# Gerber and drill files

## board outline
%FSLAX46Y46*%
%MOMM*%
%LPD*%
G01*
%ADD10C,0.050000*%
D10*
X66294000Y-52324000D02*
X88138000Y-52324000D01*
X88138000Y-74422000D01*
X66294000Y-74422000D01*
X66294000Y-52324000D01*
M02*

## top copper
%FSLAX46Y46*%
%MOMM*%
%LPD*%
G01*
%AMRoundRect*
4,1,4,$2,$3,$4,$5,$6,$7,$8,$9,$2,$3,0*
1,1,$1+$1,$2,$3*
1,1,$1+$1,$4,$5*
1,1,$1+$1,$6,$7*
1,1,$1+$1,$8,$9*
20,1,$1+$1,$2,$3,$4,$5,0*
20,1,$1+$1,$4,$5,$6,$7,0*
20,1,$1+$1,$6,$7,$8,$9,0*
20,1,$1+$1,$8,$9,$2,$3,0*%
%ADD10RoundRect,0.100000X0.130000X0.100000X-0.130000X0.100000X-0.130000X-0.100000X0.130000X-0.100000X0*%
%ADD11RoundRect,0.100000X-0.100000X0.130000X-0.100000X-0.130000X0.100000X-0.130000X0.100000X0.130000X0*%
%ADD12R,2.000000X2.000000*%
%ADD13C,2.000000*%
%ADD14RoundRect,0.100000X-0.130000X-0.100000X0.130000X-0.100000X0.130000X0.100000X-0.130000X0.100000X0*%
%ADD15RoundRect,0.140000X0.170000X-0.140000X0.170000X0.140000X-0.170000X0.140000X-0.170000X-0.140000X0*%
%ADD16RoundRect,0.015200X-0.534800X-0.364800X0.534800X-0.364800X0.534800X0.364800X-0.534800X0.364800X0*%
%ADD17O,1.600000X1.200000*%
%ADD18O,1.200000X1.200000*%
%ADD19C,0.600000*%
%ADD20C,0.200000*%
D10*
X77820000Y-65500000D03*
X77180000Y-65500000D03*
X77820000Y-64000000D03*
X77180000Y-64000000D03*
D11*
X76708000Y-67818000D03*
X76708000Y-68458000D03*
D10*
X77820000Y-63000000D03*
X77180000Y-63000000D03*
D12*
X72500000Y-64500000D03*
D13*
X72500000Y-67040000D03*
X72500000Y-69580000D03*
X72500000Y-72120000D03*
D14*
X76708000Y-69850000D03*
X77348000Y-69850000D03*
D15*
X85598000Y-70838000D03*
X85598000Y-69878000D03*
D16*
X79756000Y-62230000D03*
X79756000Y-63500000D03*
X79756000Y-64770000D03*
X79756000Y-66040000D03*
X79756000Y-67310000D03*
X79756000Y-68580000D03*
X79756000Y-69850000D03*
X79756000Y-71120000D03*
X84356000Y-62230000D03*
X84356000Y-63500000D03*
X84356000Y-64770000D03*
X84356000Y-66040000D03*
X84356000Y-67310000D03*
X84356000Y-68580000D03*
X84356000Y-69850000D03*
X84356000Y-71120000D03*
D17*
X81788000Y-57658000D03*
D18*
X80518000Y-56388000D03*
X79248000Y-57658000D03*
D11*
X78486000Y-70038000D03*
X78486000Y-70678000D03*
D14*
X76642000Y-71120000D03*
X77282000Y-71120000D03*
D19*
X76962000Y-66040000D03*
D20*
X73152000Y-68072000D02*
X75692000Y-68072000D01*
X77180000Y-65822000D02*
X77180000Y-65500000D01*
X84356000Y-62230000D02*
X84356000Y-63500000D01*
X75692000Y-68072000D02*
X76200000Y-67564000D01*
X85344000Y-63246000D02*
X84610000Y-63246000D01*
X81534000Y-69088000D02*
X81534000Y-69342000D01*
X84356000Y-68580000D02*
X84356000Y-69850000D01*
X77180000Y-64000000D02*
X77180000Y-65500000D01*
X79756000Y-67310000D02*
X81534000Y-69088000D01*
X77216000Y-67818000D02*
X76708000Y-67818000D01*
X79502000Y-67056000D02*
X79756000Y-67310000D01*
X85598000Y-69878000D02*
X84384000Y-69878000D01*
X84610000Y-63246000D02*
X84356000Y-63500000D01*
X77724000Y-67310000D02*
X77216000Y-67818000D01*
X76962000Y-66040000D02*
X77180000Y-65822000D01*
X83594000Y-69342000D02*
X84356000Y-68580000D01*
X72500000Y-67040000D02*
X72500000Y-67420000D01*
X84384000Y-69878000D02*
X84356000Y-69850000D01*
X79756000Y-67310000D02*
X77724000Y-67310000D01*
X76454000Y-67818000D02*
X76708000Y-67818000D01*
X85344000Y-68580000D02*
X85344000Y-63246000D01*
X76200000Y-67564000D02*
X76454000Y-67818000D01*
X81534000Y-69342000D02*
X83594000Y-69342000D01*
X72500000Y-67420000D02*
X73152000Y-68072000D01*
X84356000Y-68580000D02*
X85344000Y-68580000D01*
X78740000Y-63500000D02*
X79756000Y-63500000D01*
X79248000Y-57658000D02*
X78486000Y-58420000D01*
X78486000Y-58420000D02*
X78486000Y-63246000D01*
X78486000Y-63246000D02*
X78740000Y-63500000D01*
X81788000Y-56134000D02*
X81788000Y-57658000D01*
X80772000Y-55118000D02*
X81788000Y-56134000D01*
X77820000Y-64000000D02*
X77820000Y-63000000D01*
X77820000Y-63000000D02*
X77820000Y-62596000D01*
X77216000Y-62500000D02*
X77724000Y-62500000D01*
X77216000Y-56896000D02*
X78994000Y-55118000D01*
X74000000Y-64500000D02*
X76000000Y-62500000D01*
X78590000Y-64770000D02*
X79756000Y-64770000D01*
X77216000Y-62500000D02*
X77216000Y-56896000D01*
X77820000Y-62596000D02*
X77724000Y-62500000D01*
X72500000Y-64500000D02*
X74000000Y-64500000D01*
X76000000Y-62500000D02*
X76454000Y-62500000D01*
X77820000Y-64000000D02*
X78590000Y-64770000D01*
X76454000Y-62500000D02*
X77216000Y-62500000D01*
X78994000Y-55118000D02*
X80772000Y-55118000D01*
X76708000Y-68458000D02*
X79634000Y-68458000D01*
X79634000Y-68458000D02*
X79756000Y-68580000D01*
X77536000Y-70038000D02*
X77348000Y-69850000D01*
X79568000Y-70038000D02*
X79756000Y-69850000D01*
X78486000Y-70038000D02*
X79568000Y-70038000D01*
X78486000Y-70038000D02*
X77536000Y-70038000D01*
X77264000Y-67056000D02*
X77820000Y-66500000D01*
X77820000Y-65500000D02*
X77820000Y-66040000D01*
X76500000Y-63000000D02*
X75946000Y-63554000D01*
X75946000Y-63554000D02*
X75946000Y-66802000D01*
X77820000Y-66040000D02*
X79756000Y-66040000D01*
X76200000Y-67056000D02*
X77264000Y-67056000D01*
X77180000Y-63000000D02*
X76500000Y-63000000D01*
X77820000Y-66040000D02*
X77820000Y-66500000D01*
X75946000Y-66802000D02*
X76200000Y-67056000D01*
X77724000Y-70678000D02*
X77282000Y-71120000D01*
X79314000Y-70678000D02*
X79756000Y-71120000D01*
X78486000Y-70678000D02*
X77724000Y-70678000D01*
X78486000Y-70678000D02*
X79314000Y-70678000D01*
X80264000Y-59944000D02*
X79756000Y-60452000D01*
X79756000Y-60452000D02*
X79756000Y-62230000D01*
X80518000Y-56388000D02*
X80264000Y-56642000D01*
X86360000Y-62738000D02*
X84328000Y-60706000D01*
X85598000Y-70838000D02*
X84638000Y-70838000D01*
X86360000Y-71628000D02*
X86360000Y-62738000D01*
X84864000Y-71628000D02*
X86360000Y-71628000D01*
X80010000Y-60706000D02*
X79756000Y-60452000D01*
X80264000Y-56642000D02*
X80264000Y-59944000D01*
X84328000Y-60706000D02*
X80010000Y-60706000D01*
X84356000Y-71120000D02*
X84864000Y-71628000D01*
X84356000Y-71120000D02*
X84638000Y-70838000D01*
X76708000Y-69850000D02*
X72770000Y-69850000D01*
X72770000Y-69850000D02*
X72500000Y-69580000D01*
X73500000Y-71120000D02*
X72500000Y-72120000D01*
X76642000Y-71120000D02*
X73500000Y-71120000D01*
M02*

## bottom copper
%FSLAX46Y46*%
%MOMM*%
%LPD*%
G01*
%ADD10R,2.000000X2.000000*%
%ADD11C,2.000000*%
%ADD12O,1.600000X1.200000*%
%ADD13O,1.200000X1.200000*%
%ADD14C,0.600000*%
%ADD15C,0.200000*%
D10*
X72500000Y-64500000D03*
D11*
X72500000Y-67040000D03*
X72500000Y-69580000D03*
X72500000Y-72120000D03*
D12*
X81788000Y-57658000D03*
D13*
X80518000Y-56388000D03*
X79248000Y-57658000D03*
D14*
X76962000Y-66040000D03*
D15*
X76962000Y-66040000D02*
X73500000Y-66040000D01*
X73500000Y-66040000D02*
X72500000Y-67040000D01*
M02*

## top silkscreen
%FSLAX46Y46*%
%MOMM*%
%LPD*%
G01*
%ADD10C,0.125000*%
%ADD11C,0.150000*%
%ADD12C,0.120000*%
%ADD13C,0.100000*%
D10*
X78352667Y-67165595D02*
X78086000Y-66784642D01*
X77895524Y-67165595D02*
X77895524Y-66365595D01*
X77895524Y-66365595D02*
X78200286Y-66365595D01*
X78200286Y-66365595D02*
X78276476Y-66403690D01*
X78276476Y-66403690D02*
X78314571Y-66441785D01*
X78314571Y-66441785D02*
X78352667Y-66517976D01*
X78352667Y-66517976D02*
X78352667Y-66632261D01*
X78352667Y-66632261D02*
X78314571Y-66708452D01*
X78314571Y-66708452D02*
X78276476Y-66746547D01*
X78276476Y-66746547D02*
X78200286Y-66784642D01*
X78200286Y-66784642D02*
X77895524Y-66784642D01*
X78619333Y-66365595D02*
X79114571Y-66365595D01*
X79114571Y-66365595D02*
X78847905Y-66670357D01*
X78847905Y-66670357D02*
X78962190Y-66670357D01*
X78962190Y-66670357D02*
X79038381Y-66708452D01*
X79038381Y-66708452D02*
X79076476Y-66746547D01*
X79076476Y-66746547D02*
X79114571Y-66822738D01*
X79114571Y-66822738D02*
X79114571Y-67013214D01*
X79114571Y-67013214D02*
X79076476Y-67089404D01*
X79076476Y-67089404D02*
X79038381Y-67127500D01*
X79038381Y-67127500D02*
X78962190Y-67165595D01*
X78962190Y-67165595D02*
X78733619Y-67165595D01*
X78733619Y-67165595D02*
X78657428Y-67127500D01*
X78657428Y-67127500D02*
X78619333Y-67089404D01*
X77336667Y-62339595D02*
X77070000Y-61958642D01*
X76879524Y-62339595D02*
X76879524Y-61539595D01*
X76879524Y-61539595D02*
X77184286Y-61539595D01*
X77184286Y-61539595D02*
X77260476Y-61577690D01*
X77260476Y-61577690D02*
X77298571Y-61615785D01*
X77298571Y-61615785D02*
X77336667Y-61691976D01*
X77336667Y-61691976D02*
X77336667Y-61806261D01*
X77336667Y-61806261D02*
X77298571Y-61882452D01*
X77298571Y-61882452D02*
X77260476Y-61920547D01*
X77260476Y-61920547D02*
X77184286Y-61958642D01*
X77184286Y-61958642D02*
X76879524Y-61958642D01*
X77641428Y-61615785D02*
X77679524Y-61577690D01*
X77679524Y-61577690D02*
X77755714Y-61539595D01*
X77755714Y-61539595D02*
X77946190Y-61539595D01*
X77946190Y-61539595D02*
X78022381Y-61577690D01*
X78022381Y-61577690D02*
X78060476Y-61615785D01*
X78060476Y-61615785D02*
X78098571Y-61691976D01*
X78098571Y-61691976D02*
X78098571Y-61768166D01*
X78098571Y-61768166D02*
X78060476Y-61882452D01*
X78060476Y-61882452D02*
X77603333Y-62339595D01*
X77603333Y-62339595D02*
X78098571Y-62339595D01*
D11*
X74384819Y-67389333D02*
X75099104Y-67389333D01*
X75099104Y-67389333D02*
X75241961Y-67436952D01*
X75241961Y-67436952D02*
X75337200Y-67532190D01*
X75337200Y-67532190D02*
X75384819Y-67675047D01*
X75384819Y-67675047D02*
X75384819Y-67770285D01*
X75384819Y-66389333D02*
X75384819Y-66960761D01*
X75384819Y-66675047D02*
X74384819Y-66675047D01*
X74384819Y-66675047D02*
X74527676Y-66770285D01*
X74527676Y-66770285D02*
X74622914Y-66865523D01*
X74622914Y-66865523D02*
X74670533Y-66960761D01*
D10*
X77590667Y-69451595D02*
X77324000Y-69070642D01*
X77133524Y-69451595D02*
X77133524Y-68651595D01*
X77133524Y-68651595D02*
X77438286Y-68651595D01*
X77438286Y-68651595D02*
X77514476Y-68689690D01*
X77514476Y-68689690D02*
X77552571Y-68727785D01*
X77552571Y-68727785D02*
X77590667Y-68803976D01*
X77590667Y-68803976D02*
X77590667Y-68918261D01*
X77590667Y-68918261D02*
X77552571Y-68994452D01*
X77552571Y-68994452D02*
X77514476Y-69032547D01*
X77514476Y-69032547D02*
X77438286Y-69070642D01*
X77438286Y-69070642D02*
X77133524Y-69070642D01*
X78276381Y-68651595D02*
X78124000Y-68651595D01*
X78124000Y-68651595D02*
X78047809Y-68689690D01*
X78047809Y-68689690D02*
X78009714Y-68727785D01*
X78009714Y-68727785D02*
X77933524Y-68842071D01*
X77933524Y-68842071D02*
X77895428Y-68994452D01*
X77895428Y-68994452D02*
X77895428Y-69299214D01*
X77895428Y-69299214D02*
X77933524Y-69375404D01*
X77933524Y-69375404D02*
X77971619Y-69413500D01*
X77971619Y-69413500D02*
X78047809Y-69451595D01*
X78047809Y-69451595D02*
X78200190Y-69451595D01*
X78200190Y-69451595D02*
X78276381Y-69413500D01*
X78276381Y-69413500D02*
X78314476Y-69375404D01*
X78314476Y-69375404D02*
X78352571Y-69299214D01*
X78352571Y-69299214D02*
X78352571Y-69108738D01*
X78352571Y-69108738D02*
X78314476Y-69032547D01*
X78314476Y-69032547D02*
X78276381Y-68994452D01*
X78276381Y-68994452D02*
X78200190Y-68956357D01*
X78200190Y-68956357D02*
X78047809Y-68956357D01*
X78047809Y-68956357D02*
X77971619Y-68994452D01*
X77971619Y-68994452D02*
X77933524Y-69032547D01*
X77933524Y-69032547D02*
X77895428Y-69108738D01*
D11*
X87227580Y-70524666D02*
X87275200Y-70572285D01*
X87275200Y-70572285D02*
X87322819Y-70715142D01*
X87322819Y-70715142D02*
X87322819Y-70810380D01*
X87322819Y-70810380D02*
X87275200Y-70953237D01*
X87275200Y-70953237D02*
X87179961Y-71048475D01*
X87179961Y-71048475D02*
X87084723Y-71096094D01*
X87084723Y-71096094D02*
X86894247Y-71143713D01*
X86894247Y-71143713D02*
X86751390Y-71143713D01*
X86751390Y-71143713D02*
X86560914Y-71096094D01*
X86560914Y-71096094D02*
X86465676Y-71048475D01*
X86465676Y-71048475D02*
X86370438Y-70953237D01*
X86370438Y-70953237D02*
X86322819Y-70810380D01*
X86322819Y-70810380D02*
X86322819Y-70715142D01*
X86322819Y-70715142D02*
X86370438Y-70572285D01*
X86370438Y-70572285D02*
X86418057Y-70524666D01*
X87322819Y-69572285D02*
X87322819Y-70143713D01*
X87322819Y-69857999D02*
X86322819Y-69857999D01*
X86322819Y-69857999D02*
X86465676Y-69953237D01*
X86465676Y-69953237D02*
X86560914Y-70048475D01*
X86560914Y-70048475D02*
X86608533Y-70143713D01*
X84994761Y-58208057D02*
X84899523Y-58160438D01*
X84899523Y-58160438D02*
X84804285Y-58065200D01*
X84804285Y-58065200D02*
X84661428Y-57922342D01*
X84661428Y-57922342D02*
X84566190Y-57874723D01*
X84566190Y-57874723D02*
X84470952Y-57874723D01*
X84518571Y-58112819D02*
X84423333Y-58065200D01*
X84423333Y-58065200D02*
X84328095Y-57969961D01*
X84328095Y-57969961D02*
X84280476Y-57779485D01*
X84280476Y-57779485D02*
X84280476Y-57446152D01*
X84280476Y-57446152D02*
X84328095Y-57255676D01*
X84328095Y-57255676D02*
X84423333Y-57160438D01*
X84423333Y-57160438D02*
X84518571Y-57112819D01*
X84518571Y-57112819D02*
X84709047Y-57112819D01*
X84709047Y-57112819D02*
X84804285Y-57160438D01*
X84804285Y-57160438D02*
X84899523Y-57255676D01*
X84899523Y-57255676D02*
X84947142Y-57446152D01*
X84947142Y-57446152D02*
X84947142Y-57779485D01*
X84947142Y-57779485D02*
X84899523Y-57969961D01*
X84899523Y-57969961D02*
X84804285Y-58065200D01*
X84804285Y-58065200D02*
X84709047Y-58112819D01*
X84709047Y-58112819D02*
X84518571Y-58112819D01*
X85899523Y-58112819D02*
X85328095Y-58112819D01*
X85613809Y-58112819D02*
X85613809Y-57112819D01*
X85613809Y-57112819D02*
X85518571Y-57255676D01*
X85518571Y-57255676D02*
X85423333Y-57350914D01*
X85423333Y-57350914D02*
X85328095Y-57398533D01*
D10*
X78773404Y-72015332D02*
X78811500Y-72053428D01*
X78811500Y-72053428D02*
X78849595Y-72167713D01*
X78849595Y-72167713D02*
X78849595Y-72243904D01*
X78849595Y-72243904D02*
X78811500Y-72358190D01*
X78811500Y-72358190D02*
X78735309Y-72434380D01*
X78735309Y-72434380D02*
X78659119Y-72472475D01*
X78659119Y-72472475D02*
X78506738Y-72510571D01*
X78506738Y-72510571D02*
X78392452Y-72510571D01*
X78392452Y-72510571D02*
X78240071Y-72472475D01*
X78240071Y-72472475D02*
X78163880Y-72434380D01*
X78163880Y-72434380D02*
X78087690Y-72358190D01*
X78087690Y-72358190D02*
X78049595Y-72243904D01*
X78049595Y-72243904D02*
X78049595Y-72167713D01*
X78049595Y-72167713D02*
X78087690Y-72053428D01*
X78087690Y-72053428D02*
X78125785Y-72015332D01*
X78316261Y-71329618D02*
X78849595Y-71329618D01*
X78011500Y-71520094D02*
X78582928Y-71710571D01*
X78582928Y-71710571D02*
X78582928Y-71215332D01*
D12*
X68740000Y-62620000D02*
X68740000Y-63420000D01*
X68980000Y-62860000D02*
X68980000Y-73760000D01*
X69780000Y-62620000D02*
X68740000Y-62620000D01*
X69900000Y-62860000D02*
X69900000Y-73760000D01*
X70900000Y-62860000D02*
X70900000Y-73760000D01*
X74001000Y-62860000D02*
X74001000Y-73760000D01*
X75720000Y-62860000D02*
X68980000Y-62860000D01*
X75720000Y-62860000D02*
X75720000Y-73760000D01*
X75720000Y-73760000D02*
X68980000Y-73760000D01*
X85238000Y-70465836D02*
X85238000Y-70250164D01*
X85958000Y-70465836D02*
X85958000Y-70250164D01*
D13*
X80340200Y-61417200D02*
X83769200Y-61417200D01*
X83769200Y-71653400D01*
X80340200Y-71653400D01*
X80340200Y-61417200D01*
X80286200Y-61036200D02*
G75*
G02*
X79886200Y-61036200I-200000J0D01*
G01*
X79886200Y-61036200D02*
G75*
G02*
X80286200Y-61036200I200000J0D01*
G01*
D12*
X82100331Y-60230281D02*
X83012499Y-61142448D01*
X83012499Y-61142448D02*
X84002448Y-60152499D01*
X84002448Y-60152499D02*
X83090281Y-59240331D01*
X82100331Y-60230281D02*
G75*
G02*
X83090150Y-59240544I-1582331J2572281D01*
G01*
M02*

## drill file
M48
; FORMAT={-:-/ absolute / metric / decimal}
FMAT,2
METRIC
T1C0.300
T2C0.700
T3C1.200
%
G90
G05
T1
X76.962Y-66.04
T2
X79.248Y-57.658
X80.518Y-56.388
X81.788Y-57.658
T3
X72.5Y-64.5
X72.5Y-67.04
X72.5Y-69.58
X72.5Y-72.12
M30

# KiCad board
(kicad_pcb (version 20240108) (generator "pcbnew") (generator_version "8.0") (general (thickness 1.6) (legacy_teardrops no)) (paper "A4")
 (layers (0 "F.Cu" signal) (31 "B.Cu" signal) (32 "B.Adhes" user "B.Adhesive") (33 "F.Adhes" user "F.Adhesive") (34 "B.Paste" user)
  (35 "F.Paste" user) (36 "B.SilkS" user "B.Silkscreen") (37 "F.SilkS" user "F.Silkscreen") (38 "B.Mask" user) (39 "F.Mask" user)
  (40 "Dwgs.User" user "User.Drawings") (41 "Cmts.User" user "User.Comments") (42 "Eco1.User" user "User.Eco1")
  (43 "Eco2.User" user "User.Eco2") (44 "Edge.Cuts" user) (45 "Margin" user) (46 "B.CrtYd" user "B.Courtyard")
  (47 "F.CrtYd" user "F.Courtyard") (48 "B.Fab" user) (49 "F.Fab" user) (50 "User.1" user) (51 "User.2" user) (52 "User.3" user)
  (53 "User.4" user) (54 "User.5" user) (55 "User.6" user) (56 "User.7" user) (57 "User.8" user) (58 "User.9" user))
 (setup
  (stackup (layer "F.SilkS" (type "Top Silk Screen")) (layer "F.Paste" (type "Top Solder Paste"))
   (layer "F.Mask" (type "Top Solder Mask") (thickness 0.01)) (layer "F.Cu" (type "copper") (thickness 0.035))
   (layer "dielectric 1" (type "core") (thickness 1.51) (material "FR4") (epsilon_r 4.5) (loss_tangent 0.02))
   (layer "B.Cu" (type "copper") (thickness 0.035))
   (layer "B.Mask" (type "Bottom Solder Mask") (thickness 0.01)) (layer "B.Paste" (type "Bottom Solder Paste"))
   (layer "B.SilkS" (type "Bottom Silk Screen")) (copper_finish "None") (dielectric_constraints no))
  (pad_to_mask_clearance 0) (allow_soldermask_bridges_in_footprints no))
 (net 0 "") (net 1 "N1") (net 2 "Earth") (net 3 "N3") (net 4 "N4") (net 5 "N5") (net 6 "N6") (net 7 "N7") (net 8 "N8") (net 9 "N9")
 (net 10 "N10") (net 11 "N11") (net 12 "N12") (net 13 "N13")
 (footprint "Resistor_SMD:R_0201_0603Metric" (layer "F.Cu") (at 77.5 65.5 180)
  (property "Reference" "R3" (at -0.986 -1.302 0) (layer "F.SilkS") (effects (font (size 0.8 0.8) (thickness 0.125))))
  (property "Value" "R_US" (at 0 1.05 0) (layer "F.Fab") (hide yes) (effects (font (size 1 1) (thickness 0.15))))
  (pad "" smd roundrect (at -0.345 0 180) (size 0.318 0.36) (layers "F.Paste") (roundrect_rratio 0.25))
  (pad "" smd roundrect (at 0.345 0 180) (size 0.318 0.36) (layers "F.Paste") (roundrect_rratio 0.25))
  (pad "1" smd roundrect (at -0.32 0 180) (size 0.46 0.4) (layers "F.Cu" "F.Mask") (roundrect_rratio 0.25) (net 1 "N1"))
  (pad "2" smd roundrect (at 0.32 0 180) (size 0.46 0.4) (layers "F.Cu" "F.Mask") (roundrect_rratio 0.25) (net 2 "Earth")))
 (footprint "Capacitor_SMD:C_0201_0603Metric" (layer "F.Cu") (at 77.5 64 180)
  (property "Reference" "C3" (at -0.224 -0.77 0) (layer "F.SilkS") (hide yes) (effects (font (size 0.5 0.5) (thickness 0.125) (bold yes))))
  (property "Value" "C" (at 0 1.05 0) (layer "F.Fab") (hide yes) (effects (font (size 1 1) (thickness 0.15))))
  (pad "" smd roundrect (at -0.345 0 180) (size 0.318 0.36) (layers "F.Paste") (roundrect_rratio 0.25))
  (pad "" smd roundrect (at 0.345 0 180) (size 0.318 0.36) (layers "F.Paste") (roundrect_rratio 0.25))
  (pad "1" smd roundrect (at -0.32 0 180) (size 0.46 0.4) (layers "F.Cu" "F.Mask") (roundrect_rratio 0.25) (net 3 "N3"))
  (pad "2" smd roundrect (at 0.32 0 180) (size 0.46 0.4) (layers "F.Cu" "F.Mask") (roundrect_rratio 0.25) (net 2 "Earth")))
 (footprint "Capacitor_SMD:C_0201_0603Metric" (layer "F.Cu") (at 76.708 68.138 -90)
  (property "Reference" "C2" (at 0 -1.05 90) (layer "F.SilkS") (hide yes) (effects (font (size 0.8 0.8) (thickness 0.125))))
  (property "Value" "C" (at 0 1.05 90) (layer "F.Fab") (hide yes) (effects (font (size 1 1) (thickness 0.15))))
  (pad "" smd roundrect (at -0.345 0 270) (size 0.318 0.36) (layers "F.Paste") (roundrect_rratio 0.25))
  (pad "" smd roundrect (at 0.345 0 270) (size 0.318 0.36) (layers "F.Paste") (roundrect_rratio 0.25))
  (pad "1" smd roundrect (at -0.32 0 270) (size 0.46 0.4) (layers "F.Cu" "F.Mask") (roundrect_rratio 0.25) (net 2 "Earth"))
  (pad "2" smd roundrect (at 0.32 0 270) (size 0.46 0.4) (layers "F.Cu" "F.Mask") (roundrect_rratio 0.25) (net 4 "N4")))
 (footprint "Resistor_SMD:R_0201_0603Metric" (layer "F.Cu") (at 77.5 63 180)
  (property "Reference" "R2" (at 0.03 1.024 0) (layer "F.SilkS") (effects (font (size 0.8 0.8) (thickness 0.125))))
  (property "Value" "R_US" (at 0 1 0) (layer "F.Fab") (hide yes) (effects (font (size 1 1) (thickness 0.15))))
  (pad "" smd roundrect (at -0.345 0 180) (size 0.318 0.36) (layers "F.Paste") (roundrect_rratio 0.25) (clearance 0.18))
  (pad "" smd roundrect (at 0.345 0 180) (size 0.318 0.36) (layers "F.Paste") (roundrect_rratio 0.25))
  (pad "1" smd roundrect (at -0.32 0 180) (size 0.46 0.4) (layers "F.Cu" "F.Mask") (roundrect_rratio 0.25) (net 3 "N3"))
  (pad "2" smd roundrect (at 0.32 0 180) (size 0.46 0.4) (layers "F.Cu" "F.Mask") (roundrect_rratio 0.25) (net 1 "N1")))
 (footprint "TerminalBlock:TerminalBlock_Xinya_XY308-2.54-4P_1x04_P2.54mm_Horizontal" (layer "F.Cu") (at 72.5 64.5 -90)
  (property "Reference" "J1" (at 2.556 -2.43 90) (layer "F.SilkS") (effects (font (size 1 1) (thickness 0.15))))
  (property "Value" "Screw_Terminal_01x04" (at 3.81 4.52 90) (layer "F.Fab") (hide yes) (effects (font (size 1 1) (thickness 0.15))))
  (fp_line (start -1.88 3.76) (end -1.08 3.76) (stroke (width 0.12) (type solid)) (layer "F.SilkS"))
  (fp_line (start -1.64 3.52) (end 9.26 3.52) (stroke (width 0.12) (type solid)) (layer "F.SilkS"))
  (fp_line (start -1.88 2.72) (end -1.88 3.76) (stroke (width 0.12) (type solid)) (layer "F.SilkS"))
  (fp_line (start -1.64 2.6) (end 9.26 2.6) (stroke (width 0.12) (type solid)) (layer "F.SilkS"))
  (fp_line (start -1.64 1.6) (end 9.26 1.6) (stroke (width 0.12) (type solid)) (layer "F.SilkS"))
  (fp_line (start -1.64 -1.501) (end 9.26 -1.501) (stroke (width 0.12) (type solid)) (layer "F.SilkS"))
  (fp_line (start -1.64 -3.22) (end -1.64 3.52) (stroke (width 0.12) (type solid)) (layer "F.SilkS"))
  (fp_line (start -1.64 -3.22) (end 9.26 -3.22) (stroke (width 0.12) (type solid)) (layer "F.SilkS"))
  (fp_line (start 9.26 -3.22) (end 9.26 3.52) (stroke (width 0.12) (type solid)) (layer "F.SilkS"))
  (pad "1" thru_hole rect (at 0 0 270) (size 2 2) (drill 1.2) (layers "*.Cu" "*.Mask") (remove_unused_layers no) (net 3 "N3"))
  (pad "2" thru_hole circle (at 2.54 0 270) (size 2 2) (drill 1.2) (layers "*.Cu" "*.Mask") (remove_unused_layers no) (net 2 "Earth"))
  (pad "3" thru_hole circle (at 5.08 0 270) (size 2 2) (drill 1.2) (layers "*.Cu" "*.Mask") (remove_unused_layers no) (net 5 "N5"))
  (pad "4" thru_hole circle (at 7.62 0 270) (size 2 2) (drill 1.2) (layers "*.Cu" "*.Mask") (remove_unused_layers no) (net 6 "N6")))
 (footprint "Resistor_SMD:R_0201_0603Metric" (layer "F.Cu") (at 77.028 69.85)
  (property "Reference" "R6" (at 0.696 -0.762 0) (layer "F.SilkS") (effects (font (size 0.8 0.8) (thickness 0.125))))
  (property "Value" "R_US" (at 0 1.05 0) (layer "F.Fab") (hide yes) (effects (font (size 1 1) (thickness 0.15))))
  (pad "" smd roundrect (at -0.345 0) (size 0.318 0.36) (layers "F.Paste") (roundrect_rratio 0.25))
  (pad "" smd roundrect (at 0.345 0) (size 0.318 0.36) (layers "F.Paste") (roundrect_rratio 0.25))
  (pad "1" smd roundrect (at -0.32 0) (size 0.46 0.4) (layers "F.Cu" "F.Mask") (roundrect_rratio 0.25) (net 5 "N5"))
  (pad "2" smd roundrect (at 0.32 0) (size 0.46 0.4) (layers "F.Cu" "F.Mask") (roundrect_rratio 0.25) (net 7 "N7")))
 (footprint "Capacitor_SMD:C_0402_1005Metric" (layer "F.Cu") (at 85.598 70.358 90)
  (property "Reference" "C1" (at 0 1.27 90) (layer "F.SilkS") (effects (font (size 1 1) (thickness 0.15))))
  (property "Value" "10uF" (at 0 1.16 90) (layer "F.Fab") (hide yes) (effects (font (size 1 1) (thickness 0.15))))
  (fp_line (start -0.107836 -0.36) (end 0.107836 -0.36) (stroke (width 0.12) (type solid)) (layer "F.SilkS"))
  (fp_line (start -0.107836 0.36) (end 0.107836 0.36) (stroke (width 0.12) (type solid)) (layer "F.SilkS"))
  (pad "1" smd roundrect (at -0.48 0 90) (size 0.56 0.62) (layers "F.Cu" "F.Paste" "F.Mask") (roundrect_rratio 0.25) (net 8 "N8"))
  (pad "2" smd roundrect (at 0.48 0 90) (size 0.56 0.62) (layers "F.Cu" "F.Paste" "F.Mask") (roundrect_rratio 0.25) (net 2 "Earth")))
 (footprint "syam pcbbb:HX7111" (layer "F.Cu") (at 87.5792 58.2168)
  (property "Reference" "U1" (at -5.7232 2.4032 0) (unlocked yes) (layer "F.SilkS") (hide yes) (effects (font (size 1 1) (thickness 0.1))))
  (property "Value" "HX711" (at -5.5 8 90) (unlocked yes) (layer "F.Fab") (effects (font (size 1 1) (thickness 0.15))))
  (fp_rect (start -7.239 3.2004) (end -3.81 13.4366) (stroke (width 0.1) (type default)) (fill none) (layer "F.SilkS"))
  (fp_circle (center -7.493 2.8194) (end -7.293 2.8194) (stroke (width 0.1) (type default)) (fill none) (layer "F.SilkS"))
  (pad "1" smd roundrect (at -7.8232 4.0132) (size 1.1 0.76) (layers "F.Cu" "F.Paste" "F.Mask") (roundrect_rratio 0.02) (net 8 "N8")
   (thermal_bridge_angle 45))
  (pad "2" smd roundrect (at -7.8232 5.2832) (size 1.1 0.76) (layers "F.Cu" "F.Paste" "F.Mask") (roundrect_rratio 0.02) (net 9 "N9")
   (thermal_bridge_angle 45))
  (pad "3" smd roundrect (at -7.8232 6.5532) (size 1.1 0.76) (layers "F.Cu" "F.Paste" "F.Mask") (roundrect_rratio 0.02) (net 3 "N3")
   (thermal_bridge_angle 45))
  (pad "4" smd roundrect (at -7.8232 7.8232) (size 1.1 0.76) (layers "F.Cu" "F.Paste" "F.Mask") (roundrect_rratio 0.02) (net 1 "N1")
   (thermal_bridge_angle 45))
  (pad "5" smd roundrect (at -7.8232 9.0932) (size 1.1 0.76) (layers "F.Cu" "F.Paste" "F.Mask") (roundrect_rratio 0.02) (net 2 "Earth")
   (thermal_bridge_angle 45))
  (pad "6" smd roundrect (at -7.8232 10.3632) (size 1.1 0.76) (layers "F.Cu" "F.Paste" "F.Mask") (roundrect_rratio 0.02) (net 4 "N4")
   (thermal_bridge_angle 45))
  (pad "7" smd roundrect (at -7.8232 11.6332) (size 1.1 0.76) (layers "F.Cu" "F.Paste" "F.Mask") (roundrect_rratio 0.02) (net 7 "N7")
   (thermal_bridge_angle 45))
  (pad "8" smd roundrect (at -7.8232 12.9032) (size 1.1 0.76) (layers "F.Cu" "F.Paste" "F.Mask") (roundrect_rratio 0.02) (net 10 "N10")
   (thermal_bridge_angle 45))
  (pad "9" smd roundrect (at -3.2232 4.0132) (size 1.1 0.76) (layers "F.Cu" "F.Paste" "F.Mask") (roundrect_rratio 0.02) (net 2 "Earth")
   (thermal_bridge_angle 45))
  (pad "10" smd roundrect (at -3.2232 5.2832) (size 1.1 0.76) (layers "F.Cu" "F.Paste" "F.Mask") (roundrect_rratio 0.02) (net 2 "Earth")
   (thermal_bridge_angle 45))
  (pad "11" smd roundrect (at -3.2232 6.5532) (size 1.1 0.76) (layers "F.Cu" "F.Paste" "F.Mask") (roundrect_rratio 0.02) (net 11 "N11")
   (thermal_bridge_angle 45))
  (pad "12" smd roundrect (at -3.2232 7.8232) (size 1.1 0.76) (layers "F.Cu" "F.Paste" "F.Mask") (roundrect_rratio 0.02) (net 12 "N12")
   (thermal_bridge_angle 45))
  (pad "13" smd roundrect (at -3.2232 9.0932) (size 1.1 0.76) (layers "F.Cu" "F.Paste" "F.Mask") (roundrect_rratio 0.02) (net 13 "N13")
   (thermal_bridge_angle 45))
  (pad "14" smd roundrect (at -3.2232 10.3632) (size 1.1 0.76) (layers "F.Cu" "F.Paste" "F.Mask") (roundrect_rratio 0.02) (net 2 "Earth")
   (thermal_bridge_angle 45))
  (pad "15" smd roundrect (at -3.2232 11.6332) (size 1.1 0.76) (layers "F.Cu" "F.Paste" "F.Mask") (roundrect_rratio 0.02) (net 2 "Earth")
   (thermal_bridge_angle 45))
  (pad "16" smd roundrect (at -3.2232 12.9032) (size 1.1 0.76) (layers "F.Cu" "F.Paste" "F.Mask") (roundrect_rratio 0.02) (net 8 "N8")
   (thermal_bridge_angle 45)))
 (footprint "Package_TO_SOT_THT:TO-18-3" (layer "F.Cu") (at 81.788 57.658 180)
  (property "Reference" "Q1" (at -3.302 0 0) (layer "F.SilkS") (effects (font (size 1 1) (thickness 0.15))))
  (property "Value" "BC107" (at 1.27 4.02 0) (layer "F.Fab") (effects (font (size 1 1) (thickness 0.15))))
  (fp_line (start -0.312331 -2.572281) (end -1.224499 -3.484448) (stroke (width 0.12) (type solid)) (layer "F.SilkS"))
  (fp_line (start -1.224499 -3.484448) (end -2.214448 -2.494499) (stroke (width 0.12) (type solid)) (layer "F.SilkS"))
  (fp_line (start -2.214448 -2.494499) (end -1.302281 -1.582331) (stroke (width 0.12) (type solid)) (layer "F.SilkS"))
  (fp_arc (start -0.312331 -2.572281) (mid 3.405374 2.135551) (end -1.30215 -1.582544) (stroke (width 0.12) (type solid)) (layer "F.SilkS"))
  (pad "1" thru_hole oval (at 0 0 180) (size 1.6 1.2) (drill 0.7) (layers "*.Cu" "*.Mask") (remove_unused_layers no) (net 3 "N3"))
  (pad "2" thru_hole oval (at 1.27 1.27 180) (size 1.2 1.2) (drill 0.7) (layers "*.Cu" "*.Mask") (remove_unused_layers no) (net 8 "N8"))
  (pad "3" thru_hole oval (at 2.54 0 180) (size 1.2 1.2) (drill 0.7) (layers "*.Cu" "*.Mask") (remove_unused_layers no) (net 9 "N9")))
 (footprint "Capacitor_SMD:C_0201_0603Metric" (layer "F.Cu") (at 78.486 70.358 -90)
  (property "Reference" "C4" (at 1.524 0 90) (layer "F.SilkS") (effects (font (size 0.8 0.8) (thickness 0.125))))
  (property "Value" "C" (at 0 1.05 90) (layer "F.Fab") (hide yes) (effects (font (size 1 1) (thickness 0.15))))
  (pad "" smd roundrect (at -0.345 0 270) (size 0.318 0.36) (layers "F.Paste") (roundrect_rratio 0.25))
  (pad "" smd roundrect (at 0.345 0 270) (size 0.318 0.36) (layers "F.Paste") (roundrect_rratio 0.25))
  (pad "1" smd roundrect (at -0.32 0 270) (size 0.46 0.4) (layers "F.Cu" "F.Mask") (roundrect_rratio 0.25) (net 7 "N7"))
  (pad "2" smd roundrect (at 0.32 0 270) (size 0.46 0.4) (layers "F.Cu" "F.Mask") (roundrect_rratio 0.25) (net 10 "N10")))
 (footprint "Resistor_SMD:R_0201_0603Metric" (layer "F.Cu") (at 76.962 71.12)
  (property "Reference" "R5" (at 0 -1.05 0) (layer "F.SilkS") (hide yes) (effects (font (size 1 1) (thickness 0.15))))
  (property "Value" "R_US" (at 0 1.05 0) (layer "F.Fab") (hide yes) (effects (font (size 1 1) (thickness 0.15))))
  (pad "" smd roundrect (at -0.345 0) (size 0.318 0.36) (layers "F.Paste") (roundrect_rratio 0.25))
  (pad "" smd roundrect (at 0.345 0) (size 0.318 0.36) (layers "F.Paste") (roundrect_rratio 0.25))
  (pad "1" smd roundrect (at -0.32 0) (size 0.46 0.4) (layers "F.Cu" "F.Mask") (roundrect_rratio 0.25) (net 6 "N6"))
  (pad "2" smd roundrect (at 0.32 0) (size 0.46 0.4) (layers "F.Cu" "F.Mask") (roundrect_rratio 0.25) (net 10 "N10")))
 (gr_rect (start 66.294 52.324) (end 88.138 74.422) (stroke (width 0.05) (type default)) (fill none) (layer "Edge.Cuts"))
 (segment (start 73.152 68.072) (end 75.692 68.072) (width 0.2) (layer "F.Cu") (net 2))
 (segment (start 77.18 65.822) (end 77.18 65.5) (width 0.2) (layer "F.Cu") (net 2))
 (segment (start 84.356 62.23) (end 84.356 63.5) (width 0.2) (layer "F.Cu") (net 2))
 (segment (start 75.692 68.072) (end 76.2 67.564) (width 0.2) (layer "F.Cu") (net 2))
 (segment (start 85.344 63.246) (end 84.61 63.246) (width 0.2) (layer "F.Cu") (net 2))
 (segment (start 81.534 69.088) (end 81.534 69.342) (width 0.2) (layer "F.Cu") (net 2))
 (segment (start 84.356 68.58) (end 84.356 69.85) (width 0.2) (layer "F.Cu") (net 2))
 (segment (start 77.18 64) (end 77.18 65.5) (width 0.2) (layer "F.Cu") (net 2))
 (segment (start 79.756 67.31) (end 81.534 69.088) (width 0.2) (layer "F.Cu") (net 2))
 (segment (start 77.216 67.818) (end 76.708 67.818) (width 0.2) (layer "F.Cu") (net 2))
 (segment (start 79.502 67.056) (end 79.756 67.31) (width 0.2) (layer "F.Cu") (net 2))
 (segment (start 85.598 69.878) (end 84.384 69.878) (width 0.2) (layer "F.Cu") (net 2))
 (segment (start 84.61 63.246) (end 84.356 63.5) (width 0.2) (layer "F.Cu") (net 2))
 (segment (start 77.724 67.31) (end 77.216 67.818) (width 0.2) (layer "F.Cu") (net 2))
 (segment (start 76.962 66.04) (end 77.18 65.822) (width 0.2) (layer "F.Cu") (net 2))
 (segment (start 83.594 69.342) (end 84.356 68.58) (width 0.2) (layer "F.Cu") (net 2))
 (segment (start 72.5 67.04) (end 72.5 67.42) (width 0.2) (layer "F.Cu") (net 2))
 (segment (start 84.384 69.878) (end 84.356 69.85) (width 0.2) (layer "F.Cu") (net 2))
 (segment (start 79.756 67.31) (end 77.724 67.31) (width 0.2) (layer "F.Cu") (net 2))
 (segment (start 76.454 67.818) (end 76.708 67.818) (width 0.2) (layer "F.Cu") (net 2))
 (segment (start 85.344 68.58) (end 85.344 63.246) (width 0.2) (layer "F.Cu") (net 2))
 (segment (start 76.2 67.564) (end 76.454 67.818) (width 0.2) (layer "F.Cu") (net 2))
 (segment (start 81.534 69.342) (end 83.594 69.342) (width 0.2) (layer "F.Cu") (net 2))
 (segment (start 72.5 67.42) (end 73.152 68.072) (width 0.2) (layer "F.Cu") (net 2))
 (segment (start 84.356 68.58) (end 85.344 68.58) (width 0.2) (layer "F.Cu") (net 2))
 (via (at 76.962 66.04) (size 0.6) (drill 0.3) (layers "F.Cu" "B.Cu") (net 2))
 (segment (start 76.962 66.04) (end 73.5 66.04) (width 0.2) (layer "B.Cu") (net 2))
 (segment (start 73.5 66.04) (end 72.5 67.04) (width 0.2) (layer "B.Cu") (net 2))
 (segment (start 78.74 63.5) (end 79.756 63.5) (width 0.2) (layer "F.Cu") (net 9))
 (segment (start 79.248 57.658) (end 78.486 58.42) (width 0.2) (layer "F.Cu") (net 9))
 (segment (start 78.486 58.42) (end 78.486 63.246) (width 0.2) (layer "F.Cu") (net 9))
 (segment (start 78.486 63.246) (end 78.74 63.5) (width 0.2) (layer "F.Cu") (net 9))
 (segment (start 81.788 56.134) (end 81.788 57.658) (width 0.2) (layer "F.Cu") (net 3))
 (segment (start 80.772 55.118) (end 81.788 56.134) (width 0.2) (layer "F.Cu") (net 3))
 (segment (start 77.82 64) (end 77.82 63) (width 0.2) (layer "F.Cu") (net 3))
 (segment (start 77.82 63) (end 77.82 62.596) (width 0.2) (layer "F.Cu") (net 3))
 (segment (start 77.216 62.5) (end 77.724 62.5) (width 0.2) (layer "F.Cu") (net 3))
 (segment (start 77.216 56.896) (end 78.994 55.118) (width 0.2) (layer "F.Cu") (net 3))
 (segment (start 74 64.5) (end 76 62.5) (width 0.2) (layer "F.Cu") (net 3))
 (segment (start 78.59 64.77) (end 79.756 64.77) (width 0.2) (layer "F.Cu") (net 3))
 (segment (start 77.216 62.5) (end 77.216 56.896) (width 0.2) (layer "F.Cu") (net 3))
 (segment (start 77.82 62.596) (end 77.724 62.5) (width 0.2) (layer "F.Cu") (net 3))
 (segment (start 72.5 64.5) (end 74 64.5) (width 0.2) (layer "F.Cu") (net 3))
 (segment (start 76 62.5) (end 76.454 62.5) (width 0.2) (layer "F.Cu") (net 3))
 (segment (start 77.82 64) (end 78.59 64.77) (width 0.2) (layer "F.Cu") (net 3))
 (segment (start 76.454 62.5) (end 77.216 62.5) (width 0.2) (layer "F.Cu") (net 3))
 (segment (start 78.994 55.118) (end 80.772 55.118) (width 0.2) (layer "F.Cu") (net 3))
 (segment (start 76.708 68.458) (end 79.634 68.458) (width 0.2) (layer "F.Cu") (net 4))
 (segment (start 79.634 68.458) (end 79.756 68.58) (width 0.2) (layer "F.Cu") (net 4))
 (segment (start 77.536 70.038) (end 77.348 69.85) (width 0.2) (layer "F.Cu") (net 7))
 (segment (start 79.568 70.038) (end 79.756 69.85) (width 0.2) (layer "F.Cu") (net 7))
 (segment (start 78.486 70.038) (end 79.568 70.038) (width 0.2) (layer "F.Cu") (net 7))
 (segment (start 78.486 70.038) (end 77.536 70.038) (width 0.2) (layer "F.Cu") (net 7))
 (segment (start 77.264 67.056) (end 77.82 66.5) (width 0.2) (layer "F.Cu") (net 1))
 (segment (start 77.82 65.5) (end 77.82 66.04) (width 0.2) (layer "F.Cu") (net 1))
 (segment (start 76.5 63) (end 75.946 63.554) (width 0.2) (layer "F.Cu") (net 1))
 (segment (start 75.946 63.554) (end 75.946 66.802) (width 0.2) (layer "F.Cu") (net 1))
 (segment (start 77.82 66.04) (end 79.756 66.04) (width 0.2) (layer "F.Cu") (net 1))
 (segment (start 76.2 67.056) (end 77.264 67.056) (width 0.2) (layer "F.Cu") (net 1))
 (segment (start 77.18 63) (end 76.5 63) (width 0.2) (layer "F.Cu") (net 1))
 (segment (start 77.82 66.04) (end 77.82 66.5) (width 0.2) (layer "F.Cu") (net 1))
 (segment (start 75.946 66.802) (end 76.2 67.056) (width 0.2) (layer "F.Cu") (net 1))
 (segment (start 77.724 70.678) (end 77.282 71.12) (width 0.2) (layer "F.Cu") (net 10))
 (segment (start 79.314 70.678) (end 79.756 71.12) (width 0.2) (layer "F.Cu") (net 10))
 (segment (start 78.486 70.678) (end 77.724 70.678) (width 0.2) (layer "F.Cu") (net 10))
 (segment (start 78.486 70.678) (end 79.314 70.678) (width 0.2) (layer "F.Cu") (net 10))
 (segment (start 80.264 59.944) (end 79.756 60.452) (width 0.2) (layer "F.Cu") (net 8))
 (segment (start 79.756 60.452) (end 79.756 62.23) (width 0.2) (layer "F.Cu") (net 8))
 (segment (start 80.518 56.388) (end 80.264 56.642) (width 0.2) (layer "F.Cu") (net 8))
 (segment (start 86.36 62.738) (end 84.328 60.706) (width 0.2) (layer "F.Cu") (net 8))
 (segment (start 85.598 70.838) (end 84.638 70.838) (width 0.2) (layer "F.Cu") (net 8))
 (segment (start 86.36 71.628) (end 86.36 62.738) (width 0.2) (layer "F.Cu") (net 8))
 (segment (start 84.864 71.628) (end 86.36 71.628) (width 0.2) (layer "F.Cu") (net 8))
 (segment (start 80.01 60.706) (end 79.756 60.452) (width 0.2) (layer "F.Cu") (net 8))
 (segment (start 80.264 56.642) (end 80.264 59.944) (width 0.2) (layer "F.Cu") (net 8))
 (segment (start 84.328 60.706) (end 80.01 60.706) (width 0.2) (layer "F.Cu") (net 8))
 (segment (start 84.356 71.12) (end 84.864 71.628) (width 0.2) (layer "F.Cu") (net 8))
 (segment (start 84.356 71.12) (end 84.638 70.838) (width 0.2) (layer "F.Cu") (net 8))
 (segment (start 76.708 69.85) (end 72.77 69.85) (width 0.2) (layer "F.Cu") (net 5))
 (segment (start 72.77 69.85) (end 72.5 69.58) (width 0.2) (layer "F.Cu") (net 5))
 (segment (start 73.5 71.12) (end 72.5 72.12) (width 0.2) (layer "F.Cu") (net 6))
 (segment (start 76.642 71.12) (end 73.5 71.12) (width 0.2) (layer "F.Cu") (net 6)))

